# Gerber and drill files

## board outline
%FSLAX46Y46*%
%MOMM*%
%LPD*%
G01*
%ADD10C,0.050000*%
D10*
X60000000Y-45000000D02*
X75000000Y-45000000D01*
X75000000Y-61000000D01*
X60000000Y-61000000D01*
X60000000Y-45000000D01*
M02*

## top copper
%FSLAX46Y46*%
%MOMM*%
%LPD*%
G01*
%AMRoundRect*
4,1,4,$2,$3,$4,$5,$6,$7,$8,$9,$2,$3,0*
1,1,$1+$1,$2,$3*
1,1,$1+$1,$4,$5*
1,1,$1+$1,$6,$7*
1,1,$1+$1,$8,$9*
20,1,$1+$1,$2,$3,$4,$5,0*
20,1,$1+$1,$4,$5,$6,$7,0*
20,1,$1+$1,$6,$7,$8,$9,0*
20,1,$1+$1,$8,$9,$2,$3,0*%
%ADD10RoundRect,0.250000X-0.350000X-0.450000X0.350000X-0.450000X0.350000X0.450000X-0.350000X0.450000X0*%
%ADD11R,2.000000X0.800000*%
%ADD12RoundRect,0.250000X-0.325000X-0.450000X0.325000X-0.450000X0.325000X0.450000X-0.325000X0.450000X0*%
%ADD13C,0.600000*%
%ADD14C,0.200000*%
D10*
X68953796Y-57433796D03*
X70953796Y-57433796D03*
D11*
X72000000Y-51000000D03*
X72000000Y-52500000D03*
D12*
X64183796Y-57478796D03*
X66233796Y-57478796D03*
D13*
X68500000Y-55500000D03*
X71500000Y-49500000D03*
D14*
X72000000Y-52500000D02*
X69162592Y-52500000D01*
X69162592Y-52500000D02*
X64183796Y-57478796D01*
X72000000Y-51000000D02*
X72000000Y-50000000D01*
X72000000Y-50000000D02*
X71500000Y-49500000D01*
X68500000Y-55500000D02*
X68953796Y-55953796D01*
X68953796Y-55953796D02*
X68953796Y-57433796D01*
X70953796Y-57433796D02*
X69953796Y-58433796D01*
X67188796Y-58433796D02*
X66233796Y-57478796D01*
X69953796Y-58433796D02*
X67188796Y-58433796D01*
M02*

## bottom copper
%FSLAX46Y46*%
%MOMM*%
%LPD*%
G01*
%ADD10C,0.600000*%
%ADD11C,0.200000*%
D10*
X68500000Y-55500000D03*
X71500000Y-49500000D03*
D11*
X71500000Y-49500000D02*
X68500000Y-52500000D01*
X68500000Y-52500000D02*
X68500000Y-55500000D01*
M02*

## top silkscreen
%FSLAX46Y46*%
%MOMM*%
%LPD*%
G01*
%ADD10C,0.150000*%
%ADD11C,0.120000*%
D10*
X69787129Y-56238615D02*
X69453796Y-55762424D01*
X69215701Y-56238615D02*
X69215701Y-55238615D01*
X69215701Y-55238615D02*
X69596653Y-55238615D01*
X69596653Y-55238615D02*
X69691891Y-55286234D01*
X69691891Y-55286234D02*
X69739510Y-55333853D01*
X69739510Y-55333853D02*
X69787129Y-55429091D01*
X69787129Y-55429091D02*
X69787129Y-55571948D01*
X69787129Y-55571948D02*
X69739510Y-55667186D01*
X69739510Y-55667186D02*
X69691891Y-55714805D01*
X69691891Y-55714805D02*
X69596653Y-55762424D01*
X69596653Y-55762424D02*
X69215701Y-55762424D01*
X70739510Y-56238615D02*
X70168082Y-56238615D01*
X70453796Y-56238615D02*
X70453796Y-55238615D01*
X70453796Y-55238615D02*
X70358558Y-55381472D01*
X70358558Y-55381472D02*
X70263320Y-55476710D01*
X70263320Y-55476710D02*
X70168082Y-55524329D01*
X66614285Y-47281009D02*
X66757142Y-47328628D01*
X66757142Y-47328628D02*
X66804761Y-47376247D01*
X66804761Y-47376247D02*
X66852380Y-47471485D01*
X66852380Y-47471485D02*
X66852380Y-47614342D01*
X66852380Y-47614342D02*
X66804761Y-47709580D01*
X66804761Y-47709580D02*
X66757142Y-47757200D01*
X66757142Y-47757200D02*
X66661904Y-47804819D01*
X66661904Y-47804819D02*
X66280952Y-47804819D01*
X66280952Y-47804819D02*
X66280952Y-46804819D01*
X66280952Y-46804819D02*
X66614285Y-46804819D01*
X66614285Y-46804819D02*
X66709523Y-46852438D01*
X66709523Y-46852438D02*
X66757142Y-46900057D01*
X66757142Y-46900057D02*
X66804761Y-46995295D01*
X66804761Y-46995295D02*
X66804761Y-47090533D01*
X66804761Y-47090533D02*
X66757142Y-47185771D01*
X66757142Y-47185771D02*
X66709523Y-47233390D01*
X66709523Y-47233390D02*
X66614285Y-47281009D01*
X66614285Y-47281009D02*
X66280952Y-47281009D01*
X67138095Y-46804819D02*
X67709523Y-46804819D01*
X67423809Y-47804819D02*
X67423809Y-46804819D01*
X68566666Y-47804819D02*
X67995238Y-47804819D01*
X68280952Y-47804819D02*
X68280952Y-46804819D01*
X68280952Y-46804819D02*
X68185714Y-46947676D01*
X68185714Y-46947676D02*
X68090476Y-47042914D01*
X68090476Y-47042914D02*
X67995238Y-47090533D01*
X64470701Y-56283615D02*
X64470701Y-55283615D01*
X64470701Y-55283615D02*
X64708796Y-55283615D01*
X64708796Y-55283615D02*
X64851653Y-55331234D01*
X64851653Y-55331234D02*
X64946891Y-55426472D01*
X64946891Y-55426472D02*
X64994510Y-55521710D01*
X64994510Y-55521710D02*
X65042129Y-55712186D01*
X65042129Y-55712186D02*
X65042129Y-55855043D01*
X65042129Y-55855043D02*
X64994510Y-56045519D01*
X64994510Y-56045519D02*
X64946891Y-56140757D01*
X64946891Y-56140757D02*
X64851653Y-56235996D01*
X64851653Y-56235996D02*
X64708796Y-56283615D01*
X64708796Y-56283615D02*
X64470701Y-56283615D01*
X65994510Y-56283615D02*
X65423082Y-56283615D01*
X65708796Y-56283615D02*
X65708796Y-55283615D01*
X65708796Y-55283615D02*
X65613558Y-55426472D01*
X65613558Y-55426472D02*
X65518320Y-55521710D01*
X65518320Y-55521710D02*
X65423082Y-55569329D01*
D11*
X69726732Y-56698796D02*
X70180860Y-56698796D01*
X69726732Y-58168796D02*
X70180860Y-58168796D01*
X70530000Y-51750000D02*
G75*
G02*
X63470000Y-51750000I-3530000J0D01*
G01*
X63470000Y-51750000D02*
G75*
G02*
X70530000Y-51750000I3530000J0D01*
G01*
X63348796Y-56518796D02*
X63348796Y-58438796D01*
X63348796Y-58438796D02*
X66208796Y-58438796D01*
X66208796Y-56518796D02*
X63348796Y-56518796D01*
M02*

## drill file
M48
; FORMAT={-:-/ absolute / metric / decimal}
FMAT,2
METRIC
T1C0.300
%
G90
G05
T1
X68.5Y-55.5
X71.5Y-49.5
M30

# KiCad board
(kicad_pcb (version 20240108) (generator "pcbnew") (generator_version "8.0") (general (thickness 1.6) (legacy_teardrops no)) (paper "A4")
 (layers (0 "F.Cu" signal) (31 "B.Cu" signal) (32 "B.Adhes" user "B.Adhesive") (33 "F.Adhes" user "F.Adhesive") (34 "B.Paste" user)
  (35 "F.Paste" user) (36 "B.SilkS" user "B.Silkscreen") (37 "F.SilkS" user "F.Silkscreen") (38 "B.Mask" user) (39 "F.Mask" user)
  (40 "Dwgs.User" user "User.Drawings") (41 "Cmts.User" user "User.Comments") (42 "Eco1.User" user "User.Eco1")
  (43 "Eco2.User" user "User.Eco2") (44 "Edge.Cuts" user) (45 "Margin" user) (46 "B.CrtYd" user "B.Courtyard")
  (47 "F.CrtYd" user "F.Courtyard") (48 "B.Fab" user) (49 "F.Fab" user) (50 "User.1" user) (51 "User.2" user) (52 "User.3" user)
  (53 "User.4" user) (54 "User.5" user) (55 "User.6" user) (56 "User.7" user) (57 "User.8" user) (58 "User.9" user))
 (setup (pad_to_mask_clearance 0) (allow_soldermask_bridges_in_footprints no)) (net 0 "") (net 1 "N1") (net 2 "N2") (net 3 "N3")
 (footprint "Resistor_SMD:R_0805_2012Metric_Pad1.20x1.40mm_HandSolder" (layer "F.Cu") (at 69.953796 57.433796)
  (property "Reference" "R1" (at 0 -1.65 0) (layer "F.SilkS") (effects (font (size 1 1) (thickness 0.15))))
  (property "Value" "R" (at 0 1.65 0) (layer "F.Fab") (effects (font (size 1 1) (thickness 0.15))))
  (fp_line (start -0.227064 -0.735) (end 0.227064 -0.735) (stroke (width 0.12) (type solid)) (layer "F.SilkS"))
  (fp_line (start -0.227064 0.735) (end 0.227064 0.735) (stroke (width 0.12) (type solid)) (layer "F.SilkS"))
  (pad "1" smd roundrect (at -1 0) (size 1.2 1.4) (layers "F.Cu" "F.Paste" "F.Mask") (roundrect_rratio 0.208333) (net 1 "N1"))
  (pad "2" smd roundrect (at 1 0) (size 1.2 1.4) (layers "F.Cu" "F.Paste" "F.Mask") (roundrect_rratio 0.208333) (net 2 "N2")))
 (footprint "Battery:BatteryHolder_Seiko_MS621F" (layer "F.Cu") (at 72 51.75)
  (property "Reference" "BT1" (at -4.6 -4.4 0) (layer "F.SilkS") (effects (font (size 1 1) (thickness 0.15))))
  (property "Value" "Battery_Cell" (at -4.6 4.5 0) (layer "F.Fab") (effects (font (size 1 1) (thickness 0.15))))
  (fp_circle (center -5 0) (end -1.47 0) (stroke (width 0.12) (type solid)) (fill none) (layer "F.SilkS"))
  (pad "1" smd rect (at 0 -0.75) (size 2 0.8) (layers "F.Cu" "F.Paste" "F.Mask") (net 1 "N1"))
  (pad "2" smd rect (at 0 0.75) (size 2 0.8) (layers "F.Cu" "F.Paste" "F.Mask") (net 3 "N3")))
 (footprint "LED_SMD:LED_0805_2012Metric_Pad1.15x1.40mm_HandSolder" (layer "F.Cu") (at 65.208796 57.478796)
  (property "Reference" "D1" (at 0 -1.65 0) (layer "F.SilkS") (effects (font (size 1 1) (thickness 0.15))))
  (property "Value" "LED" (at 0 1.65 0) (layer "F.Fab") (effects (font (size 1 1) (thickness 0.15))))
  (fp_line (start -1.86 -0.96) (end -1.86 0.96) (stroke (width 0.12) (type solid)) (layer "F.SilkS"))
  (fp_line (start -1.86 0.96) (end 1 0.96) (stroke (width 0.12) (type solid)) (layer "F.SilkS"))
  (fp_line (start 1 -0.96) (end -1.86 -0.96) (stroke (width 0.12) (type solid)) (layer "F.SilkS"))
  (pad "1" smd roundrect (at -1.025 0) (size 1.15 1.4) (layers "F.Cu" "F.Paste" "F.Mask") (roundrect_rratio 0.217391) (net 3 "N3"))
  (pad "2" smd roundrect (at 1.025 0) (size 1.15 1.4) (layers "F.Cu" "F.Paste" "F.Mask") (roundrect_rratio 0.217391) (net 2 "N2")))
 (gr_rect (start 60 45) (end 75 61) (stroke (width 0.05) (type default)) (fill none) (layer "Edge.Cuts"))
 (segment (start 72 52.5) (end 69.162592 52.5) (width 0.2) (layer "F.Cu") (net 3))
 (segment (start 69.162592 52.5) (end 64.183796 57.478796) (width 0.2) (layer "F.Cu") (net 3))
 (segment (start 72 51) (end 72 50) (width 0.2) (layer "F.Cu") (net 1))
 (segment (start 72 50) (end 71.5 49.5) (width 0.2) (layer "F.Cu") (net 1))
 (segment (start 68.5 55.5) (end 68.953796 55.953796) (width 0.2) (layer "F.Cu") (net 1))
 (segment (start 68.953796 55.953796) (end 68.953796 57.433796) (width 0.2) (layer "F.Cu") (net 1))
 (via (at 68.5 55.5) (size 0.6) (drill 0.3) (layers "F.Cu" "B.Cu") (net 1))
 (via (at 71.5 49.5) (size 0.6) (drill 0.3) (layers "F.Cu" "B.Cu") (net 1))
 (segment (start 71.5 49.5) (end 68.5 52.5) (width 0.2) (layer "B.Cu") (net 1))
 (segment (start 68.5 52.5) (end 68.5 55.5) (width 0.2) (layer "B.Cu") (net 1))
 (segment (start 70.953796 57.433796) (end 69.953796 58.433796) (width 0.2) (layer "F.Cu") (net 2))
 (segment (start 67.188796 58.433796) (end 66.233796 57.478796) (width 0.2) (layer "F.Cu") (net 2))
 (segment (start 69.953796 58.433796) (end 67.188796 58.433796) (width 0.2) (layer "F.Cu") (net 2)))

